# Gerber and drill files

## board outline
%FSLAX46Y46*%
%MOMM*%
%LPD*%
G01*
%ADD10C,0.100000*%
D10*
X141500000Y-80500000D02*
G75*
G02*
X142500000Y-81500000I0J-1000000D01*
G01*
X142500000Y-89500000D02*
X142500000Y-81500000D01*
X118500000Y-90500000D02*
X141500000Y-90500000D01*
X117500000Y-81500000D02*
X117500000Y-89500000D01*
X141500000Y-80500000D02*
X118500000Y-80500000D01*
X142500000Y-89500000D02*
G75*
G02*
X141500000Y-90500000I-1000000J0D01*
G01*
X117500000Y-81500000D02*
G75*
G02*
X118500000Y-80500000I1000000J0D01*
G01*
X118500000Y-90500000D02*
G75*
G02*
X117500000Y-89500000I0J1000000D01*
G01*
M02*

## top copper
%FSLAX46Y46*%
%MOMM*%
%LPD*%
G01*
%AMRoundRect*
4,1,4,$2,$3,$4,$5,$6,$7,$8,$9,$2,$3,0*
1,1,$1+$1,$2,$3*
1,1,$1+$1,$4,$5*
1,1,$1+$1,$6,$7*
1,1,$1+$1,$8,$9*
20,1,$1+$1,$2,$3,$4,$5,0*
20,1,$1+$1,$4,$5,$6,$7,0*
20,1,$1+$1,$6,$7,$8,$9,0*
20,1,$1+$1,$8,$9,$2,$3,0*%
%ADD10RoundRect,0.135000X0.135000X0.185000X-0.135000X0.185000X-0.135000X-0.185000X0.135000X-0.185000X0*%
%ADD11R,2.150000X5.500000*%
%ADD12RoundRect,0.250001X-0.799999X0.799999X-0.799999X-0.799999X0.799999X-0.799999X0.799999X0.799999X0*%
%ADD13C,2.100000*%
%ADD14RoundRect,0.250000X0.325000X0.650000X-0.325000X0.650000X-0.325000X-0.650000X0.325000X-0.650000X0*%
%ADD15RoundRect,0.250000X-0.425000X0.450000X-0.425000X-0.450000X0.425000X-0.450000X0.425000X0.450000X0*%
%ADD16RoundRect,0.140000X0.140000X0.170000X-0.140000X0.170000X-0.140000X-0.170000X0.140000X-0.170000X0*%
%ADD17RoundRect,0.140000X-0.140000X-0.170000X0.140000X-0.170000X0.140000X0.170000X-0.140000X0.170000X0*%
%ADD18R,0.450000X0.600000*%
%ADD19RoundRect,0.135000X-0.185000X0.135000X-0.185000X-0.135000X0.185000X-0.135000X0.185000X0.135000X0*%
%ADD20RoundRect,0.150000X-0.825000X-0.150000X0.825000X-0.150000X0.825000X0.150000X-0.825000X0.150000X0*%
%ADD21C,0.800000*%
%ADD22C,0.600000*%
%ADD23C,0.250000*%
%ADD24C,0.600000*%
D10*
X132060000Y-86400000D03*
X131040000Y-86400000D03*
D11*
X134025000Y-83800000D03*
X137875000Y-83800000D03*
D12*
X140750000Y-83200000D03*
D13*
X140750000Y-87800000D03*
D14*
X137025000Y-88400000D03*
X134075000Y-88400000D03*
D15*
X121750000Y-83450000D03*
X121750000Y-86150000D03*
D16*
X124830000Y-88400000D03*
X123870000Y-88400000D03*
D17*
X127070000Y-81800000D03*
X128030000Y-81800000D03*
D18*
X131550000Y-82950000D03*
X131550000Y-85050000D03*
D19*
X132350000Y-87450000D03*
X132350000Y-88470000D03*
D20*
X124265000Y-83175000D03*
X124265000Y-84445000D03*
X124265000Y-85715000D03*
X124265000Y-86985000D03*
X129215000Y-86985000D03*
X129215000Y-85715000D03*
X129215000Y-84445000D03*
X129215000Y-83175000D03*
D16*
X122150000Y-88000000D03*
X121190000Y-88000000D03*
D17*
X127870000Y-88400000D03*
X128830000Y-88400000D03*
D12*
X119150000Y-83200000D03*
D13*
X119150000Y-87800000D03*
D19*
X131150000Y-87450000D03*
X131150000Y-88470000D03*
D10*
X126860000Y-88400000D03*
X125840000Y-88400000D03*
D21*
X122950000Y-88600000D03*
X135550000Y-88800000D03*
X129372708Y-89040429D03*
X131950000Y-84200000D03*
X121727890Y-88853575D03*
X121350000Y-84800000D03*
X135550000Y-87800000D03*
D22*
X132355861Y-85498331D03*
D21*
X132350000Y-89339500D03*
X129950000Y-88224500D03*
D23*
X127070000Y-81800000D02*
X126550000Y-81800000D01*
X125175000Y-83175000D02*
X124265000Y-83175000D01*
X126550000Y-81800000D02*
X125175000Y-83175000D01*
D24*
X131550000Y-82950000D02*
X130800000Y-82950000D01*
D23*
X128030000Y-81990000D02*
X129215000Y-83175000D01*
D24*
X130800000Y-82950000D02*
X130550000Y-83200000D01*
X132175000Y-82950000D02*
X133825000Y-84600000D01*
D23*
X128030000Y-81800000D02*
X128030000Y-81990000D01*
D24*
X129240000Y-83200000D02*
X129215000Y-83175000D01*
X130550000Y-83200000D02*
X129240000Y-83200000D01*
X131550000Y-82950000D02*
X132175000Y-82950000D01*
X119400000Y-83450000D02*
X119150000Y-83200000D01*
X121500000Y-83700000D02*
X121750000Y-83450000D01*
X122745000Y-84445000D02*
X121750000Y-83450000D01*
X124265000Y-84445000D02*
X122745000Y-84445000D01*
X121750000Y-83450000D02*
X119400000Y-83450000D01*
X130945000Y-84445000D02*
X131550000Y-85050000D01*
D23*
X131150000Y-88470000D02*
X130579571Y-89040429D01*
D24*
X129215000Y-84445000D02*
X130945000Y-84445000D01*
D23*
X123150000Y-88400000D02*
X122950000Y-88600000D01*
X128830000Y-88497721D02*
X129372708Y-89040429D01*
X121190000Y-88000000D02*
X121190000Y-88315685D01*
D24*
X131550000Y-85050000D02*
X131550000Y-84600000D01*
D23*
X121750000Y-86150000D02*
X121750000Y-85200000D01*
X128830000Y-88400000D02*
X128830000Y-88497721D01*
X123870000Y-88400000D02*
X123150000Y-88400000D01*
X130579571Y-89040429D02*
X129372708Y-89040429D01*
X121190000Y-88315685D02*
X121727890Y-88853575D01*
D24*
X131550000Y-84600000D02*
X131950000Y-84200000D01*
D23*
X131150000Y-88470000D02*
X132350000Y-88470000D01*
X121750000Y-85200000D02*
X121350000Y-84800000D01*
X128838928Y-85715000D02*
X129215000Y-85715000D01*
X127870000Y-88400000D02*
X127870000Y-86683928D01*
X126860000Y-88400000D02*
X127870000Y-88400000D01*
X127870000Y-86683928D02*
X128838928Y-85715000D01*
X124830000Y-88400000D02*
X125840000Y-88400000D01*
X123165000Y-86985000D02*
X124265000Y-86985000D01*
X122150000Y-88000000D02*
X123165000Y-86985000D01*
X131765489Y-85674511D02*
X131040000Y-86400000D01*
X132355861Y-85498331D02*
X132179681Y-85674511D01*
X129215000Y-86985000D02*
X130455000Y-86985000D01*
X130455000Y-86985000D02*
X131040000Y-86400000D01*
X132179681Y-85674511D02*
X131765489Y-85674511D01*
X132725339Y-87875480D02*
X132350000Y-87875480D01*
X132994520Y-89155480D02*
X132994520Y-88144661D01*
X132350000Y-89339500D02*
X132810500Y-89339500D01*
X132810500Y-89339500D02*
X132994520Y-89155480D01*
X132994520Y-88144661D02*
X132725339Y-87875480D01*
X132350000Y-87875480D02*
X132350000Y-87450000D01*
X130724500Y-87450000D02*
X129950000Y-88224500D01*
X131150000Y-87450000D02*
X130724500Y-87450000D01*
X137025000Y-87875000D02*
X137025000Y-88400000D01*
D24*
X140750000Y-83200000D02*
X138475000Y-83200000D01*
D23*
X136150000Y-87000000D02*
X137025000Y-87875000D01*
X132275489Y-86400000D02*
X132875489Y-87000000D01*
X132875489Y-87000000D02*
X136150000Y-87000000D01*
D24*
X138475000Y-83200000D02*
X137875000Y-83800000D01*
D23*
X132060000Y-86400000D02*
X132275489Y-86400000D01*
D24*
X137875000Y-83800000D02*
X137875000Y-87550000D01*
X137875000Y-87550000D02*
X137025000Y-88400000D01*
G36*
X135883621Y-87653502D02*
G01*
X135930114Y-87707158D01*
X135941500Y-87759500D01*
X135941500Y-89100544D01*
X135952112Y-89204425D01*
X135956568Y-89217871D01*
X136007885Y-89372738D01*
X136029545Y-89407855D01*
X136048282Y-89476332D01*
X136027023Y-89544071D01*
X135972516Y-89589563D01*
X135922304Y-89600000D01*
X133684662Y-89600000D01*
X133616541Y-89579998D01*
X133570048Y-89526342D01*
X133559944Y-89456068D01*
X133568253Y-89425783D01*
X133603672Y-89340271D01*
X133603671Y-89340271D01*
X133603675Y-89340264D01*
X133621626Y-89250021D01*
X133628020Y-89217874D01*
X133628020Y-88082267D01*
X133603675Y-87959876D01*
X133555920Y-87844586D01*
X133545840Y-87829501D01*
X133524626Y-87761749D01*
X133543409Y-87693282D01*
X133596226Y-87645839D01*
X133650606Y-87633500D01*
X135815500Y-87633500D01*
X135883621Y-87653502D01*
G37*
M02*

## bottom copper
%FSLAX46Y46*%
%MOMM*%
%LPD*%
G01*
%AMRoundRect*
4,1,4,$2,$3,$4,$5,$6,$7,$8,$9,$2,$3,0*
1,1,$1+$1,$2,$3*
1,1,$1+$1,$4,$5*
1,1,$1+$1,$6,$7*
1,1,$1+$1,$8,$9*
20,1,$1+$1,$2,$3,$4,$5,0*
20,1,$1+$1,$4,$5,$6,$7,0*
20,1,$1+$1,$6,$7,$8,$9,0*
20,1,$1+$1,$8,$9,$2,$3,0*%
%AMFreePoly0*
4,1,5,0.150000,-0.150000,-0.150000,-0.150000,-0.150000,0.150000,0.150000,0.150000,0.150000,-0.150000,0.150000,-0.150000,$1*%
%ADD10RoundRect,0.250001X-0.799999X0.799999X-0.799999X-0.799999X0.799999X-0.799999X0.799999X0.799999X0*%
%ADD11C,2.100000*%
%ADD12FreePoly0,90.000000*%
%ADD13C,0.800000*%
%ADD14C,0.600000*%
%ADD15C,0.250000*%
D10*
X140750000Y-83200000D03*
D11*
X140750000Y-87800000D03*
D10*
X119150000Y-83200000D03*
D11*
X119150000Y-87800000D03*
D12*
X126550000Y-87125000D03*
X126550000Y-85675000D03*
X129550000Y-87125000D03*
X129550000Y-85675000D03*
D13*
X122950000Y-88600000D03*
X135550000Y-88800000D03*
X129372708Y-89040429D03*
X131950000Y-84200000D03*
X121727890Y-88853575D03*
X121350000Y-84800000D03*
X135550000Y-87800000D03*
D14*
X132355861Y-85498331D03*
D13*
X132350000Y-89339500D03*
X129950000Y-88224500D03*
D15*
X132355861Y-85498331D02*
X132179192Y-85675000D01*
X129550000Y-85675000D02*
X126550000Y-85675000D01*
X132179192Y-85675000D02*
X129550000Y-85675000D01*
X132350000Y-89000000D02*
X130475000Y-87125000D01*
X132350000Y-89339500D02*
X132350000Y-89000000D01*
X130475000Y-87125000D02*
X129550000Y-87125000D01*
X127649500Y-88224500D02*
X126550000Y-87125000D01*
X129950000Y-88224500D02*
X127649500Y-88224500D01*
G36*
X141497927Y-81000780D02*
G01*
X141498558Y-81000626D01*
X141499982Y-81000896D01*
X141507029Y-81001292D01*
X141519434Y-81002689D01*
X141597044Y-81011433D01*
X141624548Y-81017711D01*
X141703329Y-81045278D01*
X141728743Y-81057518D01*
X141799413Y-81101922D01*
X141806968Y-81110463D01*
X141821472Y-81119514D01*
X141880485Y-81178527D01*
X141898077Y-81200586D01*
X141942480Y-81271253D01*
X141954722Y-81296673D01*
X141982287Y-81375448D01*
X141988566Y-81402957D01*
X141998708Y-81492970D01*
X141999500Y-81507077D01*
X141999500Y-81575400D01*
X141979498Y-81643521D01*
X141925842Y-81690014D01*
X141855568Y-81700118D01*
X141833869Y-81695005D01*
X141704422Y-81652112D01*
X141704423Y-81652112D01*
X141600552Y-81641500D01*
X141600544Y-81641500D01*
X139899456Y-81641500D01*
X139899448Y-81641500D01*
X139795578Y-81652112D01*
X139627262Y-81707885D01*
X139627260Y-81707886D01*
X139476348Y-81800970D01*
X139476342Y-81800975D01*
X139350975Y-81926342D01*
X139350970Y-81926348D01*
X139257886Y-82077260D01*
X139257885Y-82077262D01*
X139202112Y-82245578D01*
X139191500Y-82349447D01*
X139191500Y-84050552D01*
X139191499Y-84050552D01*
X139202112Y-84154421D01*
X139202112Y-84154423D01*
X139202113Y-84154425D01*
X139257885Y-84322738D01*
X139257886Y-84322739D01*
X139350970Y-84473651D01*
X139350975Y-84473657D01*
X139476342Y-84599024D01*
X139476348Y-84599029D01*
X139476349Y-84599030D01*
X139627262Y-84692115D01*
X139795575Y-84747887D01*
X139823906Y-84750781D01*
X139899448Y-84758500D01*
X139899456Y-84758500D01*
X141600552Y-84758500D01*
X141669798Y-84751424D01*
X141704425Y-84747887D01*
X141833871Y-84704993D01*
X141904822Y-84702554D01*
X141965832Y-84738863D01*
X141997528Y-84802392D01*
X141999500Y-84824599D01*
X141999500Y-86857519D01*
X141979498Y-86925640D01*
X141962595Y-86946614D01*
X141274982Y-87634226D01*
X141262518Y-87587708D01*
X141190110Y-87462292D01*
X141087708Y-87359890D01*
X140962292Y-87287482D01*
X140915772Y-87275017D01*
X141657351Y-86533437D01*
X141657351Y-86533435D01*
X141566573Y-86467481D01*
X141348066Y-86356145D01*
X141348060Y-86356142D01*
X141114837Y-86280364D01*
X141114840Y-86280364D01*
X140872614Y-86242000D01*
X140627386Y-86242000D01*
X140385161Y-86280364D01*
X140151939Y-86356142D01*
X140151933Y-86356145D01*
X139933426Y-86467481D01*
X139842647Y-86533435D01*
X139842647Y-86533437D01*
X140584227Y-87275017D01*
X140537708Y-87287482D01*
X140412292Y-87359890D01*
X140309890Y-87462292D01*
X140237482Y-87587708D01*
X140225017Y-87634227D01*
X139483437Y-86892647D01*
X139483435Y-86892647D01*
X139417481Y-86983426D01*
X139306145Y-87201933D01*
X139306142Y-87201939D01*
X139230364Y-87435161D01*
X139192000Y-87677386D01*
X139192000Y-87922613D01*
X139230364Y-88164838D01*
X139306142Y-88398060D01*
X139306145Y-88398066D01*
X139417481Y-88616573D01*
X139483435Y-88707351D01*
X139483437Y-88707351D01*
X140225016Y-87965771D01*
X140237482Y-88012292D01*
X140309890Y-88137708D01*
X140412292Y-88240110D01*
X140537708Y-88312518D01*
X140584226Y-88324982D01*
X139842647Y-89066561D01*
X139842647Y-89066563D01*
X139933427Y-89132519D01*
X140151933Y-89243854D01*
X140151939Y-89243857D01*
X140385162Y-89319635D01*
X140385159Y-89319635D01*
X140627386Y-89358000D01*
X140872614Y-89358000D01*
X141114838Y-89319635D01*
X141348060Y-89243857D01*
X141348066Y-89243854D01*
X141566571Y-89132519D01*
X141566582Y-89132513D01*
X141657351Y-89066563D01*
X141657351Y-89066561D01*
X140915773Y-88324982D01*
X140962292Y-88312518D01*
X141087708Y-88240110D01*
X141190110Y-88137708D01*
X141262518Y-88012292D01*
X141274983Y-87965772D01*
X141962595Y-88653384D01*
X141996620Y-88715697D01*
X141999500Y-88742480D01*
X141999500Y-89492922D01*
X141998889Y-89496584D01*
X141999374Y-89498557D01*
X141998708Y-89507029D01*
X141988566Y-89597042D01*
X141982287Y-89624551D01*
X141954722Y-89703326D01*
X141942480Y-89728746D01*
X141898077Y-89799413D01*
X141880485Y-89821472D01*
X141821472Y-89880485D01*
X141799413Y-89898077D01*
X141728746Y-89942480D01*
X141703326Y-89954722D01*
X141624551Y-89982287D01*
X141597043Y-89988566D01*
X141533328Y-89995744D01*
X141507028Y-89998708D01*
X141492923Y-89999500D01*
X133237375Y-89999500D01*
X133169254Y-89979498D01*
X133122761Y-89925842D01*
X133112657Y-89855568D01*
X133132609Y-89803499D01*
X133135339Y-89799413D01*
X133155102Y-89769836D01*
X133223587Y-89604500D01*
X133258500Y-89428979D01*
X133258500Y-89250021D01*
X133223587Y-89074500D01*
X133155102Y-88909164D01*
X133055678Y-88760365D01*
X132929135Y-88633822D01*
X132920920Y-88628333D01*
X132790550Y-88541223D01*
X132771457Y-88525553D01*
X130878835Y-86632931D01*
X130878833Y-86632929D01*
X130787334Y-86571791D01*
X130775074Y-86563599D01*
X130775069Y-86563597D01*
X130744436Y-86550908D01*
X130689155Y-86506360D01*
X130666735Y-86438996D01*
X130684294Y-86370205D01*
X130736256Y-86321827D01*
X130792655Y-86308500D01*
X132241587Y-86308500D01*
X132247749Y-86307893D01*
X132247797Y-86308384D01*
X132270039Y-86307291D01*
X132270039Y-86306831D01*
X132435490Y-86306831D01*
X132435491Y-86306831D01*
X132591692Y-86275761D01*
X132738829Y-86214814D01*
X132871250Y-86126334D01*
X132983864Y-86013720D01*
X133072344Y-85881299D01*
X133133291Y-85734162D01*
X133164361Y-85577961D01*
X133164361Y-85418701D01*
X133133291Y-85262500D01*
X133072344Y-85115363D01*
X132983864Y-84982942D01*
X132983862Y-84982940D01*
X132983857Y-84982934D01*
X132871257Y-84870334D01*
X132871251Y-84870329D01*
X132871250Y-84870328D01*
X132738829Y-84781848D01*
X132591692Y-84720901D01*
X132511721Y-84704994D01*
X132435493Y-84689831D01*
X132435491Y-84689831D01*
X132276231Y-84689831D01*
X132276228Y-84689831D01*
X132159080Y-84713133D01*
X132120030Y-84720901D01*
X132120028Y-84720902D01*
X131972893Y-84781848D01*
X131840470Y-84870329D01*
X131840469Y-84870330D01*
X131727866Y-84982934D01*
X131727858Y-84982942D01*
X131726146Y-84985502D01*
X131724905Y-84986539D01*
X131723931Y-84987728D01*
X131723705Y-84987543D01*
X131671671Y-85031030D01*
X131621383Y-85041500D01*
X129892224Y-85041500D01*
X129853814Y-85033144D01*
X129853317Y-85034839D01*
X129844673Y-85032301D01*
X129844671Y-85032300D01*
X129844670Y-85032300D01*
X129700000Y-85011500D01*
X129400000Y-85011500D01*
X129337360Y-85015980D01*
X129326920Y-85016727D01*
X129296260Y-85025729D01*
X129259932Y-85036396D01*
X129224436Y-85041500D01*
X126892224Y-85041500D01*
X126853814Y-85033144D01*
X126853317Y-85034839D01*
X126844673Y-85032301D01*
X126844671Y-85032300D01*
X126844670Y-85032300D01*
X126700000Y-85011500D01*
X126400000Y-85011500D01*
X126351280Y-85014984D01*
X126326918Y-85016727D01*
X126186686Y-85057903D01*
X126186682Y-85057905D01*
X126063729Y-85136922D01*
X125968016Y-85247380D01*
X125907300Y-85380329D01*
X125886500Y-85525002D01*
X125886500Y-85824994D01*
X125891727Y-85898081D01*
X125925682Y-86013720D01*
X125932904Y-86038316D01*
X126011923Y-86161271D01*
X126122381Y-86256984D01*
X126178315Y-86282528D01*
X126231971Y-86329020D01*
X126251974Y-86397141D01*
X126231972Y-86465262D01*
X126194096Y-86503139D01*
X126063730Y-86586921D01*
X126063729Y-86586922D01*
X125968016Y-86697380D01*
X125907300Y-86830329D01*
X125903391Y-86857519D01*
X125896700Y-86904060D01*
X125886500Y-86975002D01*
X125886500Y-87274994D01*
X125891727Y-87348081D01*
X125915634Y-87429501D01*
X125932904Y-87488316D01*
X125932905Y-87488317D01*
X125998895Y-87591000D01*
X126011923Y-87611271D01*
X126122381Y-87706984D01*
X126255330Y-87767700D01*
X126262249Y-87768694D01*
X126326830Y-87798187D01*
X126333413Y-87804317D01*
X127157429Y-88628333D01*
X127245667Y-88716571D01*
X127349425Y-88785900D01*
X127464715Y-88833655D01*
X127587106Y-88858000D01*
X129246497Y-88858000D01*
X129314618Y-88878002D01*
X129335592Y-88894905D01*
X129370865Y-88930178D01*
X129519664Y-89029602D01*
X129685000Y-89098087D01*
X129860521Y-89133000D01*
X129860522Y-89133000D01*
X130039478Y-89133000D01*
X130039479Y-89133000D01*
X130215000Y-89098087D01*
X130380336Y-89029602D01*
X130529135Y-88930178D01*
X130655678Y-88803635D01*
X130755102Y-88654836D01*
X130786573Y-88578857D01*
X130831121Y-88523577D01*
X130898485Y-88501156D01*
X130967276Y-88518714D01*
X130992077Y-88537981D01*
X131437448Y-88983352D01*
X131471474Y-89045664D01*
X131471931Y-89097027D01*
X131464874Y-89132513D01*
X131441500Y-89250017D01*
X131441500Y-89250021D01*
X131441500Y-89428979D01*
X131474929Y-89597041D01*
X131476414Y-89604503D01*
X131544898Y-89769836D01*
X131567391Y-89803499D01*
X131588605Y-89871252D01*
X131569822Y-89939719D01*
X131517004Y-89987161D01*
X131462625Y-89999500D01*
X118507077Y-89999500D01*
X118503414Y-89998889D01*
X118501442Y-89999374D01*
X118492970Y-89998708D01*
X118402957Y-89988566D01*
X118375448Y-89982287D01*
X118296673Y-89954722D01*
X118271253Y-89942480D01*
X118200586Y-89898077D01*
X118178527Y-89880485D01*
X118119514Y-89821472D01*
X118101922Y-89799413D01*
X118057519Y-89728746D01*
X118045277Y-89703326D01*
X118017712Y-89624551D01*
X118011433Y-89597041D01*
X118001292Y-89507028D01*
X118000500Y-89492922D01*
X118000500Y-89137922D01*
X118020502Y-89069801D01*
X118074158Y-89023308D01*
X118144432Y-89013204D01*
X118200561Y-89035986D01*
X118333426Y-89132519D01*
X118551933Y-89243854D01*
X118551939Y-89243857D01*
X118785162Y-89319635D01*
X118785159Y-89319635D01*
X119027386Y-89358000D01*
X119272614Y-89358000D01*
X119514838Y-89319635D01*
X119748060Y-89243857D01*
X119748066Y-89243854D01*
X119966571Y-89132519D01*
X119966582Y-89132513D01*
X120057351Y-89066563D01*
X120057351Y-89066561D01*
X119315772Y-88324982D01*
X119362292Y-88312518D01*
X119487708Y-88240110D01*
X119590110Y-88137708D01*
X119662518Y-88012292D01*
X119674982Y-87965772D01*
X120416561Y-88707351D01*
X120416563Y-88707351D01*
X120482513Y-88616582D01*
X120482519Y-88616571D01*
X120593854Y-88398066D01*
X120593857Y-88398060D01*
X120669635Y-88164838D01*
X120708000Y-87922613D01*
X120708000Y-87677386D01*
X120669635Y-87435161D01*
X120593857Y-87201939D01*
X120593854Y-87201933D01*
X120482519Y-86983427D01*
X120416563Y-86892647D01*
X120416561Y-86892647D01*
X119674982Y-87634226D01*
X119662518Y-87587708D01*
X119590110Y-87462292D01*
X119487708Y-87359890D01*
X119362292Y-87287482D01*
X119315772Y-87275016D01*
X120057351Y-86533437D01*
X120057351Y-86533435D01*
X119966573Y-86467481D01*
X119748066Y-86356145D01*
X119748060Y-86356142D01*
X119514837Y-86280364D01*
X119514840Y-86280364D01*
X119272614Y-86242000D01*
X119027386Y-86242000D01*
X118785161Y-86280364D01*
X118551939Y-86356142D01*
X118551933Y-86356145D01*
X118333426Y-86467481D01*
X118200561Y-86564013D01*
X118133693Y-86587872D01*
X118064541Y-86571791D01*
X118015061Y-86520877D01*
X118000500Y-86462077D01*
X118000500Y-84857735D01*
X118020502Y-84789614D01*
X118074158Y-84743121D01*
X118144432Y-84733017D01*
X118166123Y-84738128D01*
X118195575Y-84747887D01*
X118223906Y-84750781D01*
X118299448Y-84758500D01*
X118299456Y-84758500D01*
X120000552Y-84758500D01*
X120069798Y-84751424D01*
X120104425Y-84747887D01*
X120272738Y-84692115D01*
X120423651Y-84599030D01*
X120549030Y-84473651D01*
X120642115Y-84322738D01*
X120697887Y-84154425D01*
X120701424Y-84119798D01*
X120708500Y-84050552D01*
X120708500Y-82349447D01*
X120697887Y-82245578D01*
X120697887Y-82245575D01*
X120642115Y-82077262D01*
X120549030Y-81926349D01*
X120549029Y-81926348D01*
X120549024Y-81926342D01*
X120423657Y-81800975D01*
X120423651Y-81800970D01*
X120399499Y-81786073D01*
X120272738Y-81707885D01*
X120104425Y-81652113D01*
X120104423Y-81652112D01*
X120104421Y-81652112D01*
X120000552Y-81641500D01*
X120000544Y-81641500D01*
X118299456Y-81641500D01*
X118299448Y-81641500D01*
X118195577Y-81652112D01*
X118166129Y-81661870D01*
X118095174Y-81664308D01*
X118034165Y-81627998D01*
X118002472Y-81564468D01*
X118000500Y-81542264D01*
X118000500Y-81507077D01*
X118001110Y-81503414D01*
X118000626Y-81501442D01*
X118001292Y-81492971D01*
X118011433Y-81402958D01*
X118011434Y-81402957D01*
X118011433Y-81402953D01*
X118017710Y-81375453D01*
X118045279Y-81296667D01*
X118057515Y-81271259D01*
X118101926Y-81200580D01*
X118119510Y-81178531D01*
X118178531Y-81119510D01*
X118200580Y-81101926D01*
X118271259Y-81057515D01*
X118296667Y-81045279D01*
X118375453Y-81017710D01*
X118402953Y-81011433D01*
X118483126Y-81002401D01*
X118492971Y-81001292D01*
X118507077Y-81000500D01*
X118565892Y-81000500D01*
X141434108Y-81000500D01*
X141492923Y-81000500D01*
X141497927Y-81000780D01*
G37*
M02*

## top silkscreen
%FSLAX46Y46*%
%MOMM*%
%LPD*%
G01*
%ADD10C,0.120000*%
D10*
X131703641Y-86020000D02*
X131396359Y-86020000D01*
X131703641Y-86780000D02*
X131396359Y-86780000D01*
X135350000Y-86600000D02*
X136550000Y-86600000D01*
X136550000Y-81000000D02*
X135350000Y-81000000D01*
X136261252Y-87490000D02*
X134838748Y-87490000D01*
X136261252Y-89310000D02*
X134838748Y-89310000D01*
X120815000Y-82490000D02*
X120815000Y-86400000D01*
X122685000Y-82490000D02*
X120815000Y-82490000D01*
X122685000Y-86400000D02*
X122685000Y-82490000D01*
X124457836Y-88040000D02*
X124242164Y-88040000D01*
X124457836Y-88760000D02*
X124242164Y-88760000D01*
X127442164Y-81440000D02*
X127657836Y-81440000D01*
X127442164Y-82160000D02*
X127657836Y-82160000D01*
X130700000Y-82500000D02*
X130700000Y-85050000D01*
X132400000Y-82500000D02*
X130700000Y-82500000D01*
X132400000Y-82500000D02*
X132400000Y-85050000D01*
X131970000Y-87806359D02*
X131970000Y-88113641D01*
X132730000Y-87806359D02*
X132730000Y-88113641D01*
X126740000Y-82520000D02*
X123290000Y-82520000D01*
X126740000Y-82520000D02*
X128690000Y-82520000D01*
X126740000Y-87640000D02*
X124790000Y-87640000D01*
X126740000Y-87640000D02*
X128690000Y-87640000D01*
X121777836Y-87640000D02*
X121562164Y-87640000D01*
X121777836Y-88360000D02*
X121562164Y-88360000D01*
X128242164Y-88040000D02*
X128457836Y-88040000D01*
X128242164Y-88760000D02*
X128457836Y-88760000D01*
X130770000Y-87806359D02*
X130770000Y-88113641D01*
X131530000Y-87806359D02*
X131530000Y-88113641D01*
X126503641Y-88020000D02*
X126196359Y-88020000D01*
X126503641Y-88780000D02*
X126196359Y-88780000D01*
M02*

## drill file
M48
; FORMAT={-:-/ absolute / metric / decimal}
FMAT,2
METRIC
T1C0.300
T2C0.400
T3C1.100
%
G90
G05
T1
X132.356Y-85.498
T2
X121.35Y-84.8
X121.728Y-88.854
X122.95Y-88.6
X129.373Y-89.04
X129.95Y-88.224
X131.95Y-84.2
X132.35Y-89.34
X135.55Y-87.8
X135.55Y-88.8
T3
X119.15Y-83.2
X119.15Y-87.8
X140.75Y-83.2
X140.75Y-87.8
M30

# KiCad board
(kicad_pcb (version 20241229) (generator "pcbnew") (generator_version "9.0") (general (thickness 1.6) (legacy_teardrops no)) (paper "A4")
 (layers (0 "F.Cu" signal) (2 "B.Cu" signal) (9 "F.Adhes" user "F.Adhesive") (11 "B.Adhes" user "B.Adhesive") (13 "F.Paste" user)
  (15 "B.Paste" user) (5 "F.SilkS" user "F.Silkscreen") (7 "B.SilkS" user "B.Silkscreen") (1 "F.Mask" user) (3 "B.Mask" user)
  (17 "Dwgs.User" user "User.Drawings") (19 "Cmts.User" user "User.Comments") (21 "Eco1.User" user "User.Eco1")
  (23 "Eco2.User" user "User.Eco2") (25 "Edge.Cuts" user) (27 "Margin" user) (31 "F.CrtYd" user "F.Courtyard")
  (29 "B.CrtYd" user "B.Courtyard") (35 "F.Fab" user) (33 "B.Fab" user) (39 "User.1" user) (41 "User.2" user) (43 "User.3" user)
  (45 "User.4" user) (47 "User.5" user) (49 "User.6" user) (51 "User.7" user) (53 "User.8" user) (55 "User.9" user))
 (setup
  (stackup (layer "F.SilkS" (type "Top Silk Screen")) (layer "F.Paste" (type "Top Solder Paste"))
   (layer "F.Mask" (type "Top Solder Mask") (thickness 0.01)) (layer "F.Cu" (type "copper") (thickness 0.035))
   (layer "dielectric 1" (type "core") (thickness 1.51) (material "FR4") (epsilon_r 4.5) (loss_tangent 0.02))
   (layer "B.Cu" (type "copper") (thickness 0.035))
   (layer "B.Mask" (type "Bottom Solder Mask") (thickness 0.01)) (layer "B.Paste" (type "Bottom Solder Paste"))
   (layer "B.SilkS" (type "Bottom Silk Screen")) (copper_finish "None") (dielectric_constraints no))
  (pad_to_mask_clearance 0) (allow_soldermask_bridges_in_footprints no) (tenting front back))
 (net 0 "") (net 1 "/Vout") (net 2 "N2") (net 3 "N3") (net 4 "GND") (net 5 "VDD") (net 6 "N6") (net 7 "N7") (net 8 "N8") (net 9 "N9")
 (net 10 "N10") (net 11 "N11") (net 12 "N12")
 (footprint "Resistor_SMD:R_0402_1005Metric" (layer "F.Cu") (at 131.55 86.4 180)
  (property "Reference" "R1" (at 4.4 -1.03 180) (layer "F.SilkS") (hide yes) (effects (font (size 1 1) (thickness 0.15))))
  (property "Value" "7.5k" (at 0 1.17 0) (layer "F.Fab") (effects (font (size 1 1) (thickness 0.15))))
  (fp_line (start -0.153641 0.38) (end 0.153641 0.38) (stroke (width 0.12) (type solid)) (layer "F.SilkS"))
  (fp_line (start -0.153641 -0.38) (end 0.153641 -0.38) (stroke (width 0.12) (type solid)) (layer "F.SilkS"))
  (pad "1" smd roundrect (at -0.51 0 180) (size 0.54 0.64) (layers "F.Cu" "F.Mask" "F.Paste") (roundrect_rratio 0.25) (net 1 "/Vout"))
  (pad "2" smd roundrect (at 0.51 0 180) (size 0.54 0.64) (layers "F.Cu" "F.Mask" "F.Paste") (roundrect_rratio 0.25) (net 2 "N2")))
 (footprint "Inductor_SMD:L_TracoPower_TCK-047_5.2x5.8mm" (layer "F.Cu") (at 135.95 83.8)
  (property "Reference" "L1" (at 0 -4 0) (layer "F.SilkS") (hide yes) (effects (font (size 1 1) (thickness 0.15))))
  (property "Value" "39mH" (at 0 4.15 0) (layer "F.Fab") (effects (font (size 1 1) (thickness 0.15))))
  (fp_line (start -0.6 2.8) (end 0.6 2.8) (stroke (width 0.12) (type solid)) (layer "F.SilkS"))
  (fp_line (start 0.6 -2.8) (end -0.6 -2.8) (stroke (width 0.12) (type solid)) (layer "F.SilkS"))
  (pad "1" smd rect (at -1.925 0 90) (size 5.5 2.15) (layers "F.Cu" "F.Mask" "F.Paste") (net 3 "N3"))
  (pad "2" smd rect (at 1.925 0 90) (size 5.5 2.15) (layers "F.Cu" "F.Mask" "F.Paste") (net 1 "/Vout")))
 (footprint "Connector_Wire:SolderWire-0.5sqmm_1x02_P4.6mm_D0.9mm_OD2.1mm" (layer "F.Cu") (at 140.75 83.2 -90)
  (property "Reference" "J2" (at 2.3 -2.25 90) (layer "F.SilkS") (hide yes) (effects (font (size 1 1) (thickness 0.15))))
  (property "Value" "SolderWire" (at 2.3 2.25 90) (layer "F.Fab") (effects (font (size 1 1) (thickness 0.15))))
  (pad "1" thru_hole roundrect (at 0 0 270) (size 2.1 2.1) (drill 1.1) (layers "*.Cu" "*.Mask") (remove_unused_layers no)
   (roundrect_rratio 0.1190480952) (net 1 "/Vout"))
  (pad "2" thru_hole circle (at 4.6 0 270) (size 2.1 2.1) (drill 1.1) (layers "*.Cu" "*.Mask") (remove_unused_layers no) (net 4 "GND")))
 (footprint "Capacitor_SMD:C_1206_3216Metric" (layer "F.Cu") (at 135.55 88.4 180)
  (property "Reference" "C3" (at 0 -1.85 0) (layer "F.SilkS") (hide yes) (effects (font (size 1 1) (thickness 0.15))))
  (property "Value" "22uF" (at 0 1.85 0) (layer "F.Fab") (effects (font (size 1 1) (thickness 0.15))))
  (fp_line (start -0.711252 0.91) (end 0.711252 0.91) (stroke (width 0.12) (type solid)) (layer "F.SilkS"))
  (fp_line (start -0.711252 -0.91) (end 0.711252 -0.91) (stroke (width 0.12) (type solid)) (layer "F.SilkS"))
  (pad "1" smd roundrect (at -1.475 0 180) (size 1.15 1.8) (layers "F.Cu" "F.Mask" "F.Paste") (roundrect_rratio 0.2173913043)
   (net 1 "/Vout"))
  (pad "2" smd roundrect (at 1.475 0 180) (size 1.15 1.8) (layers "F.Cu" "F.Mask" "F.Paste") (roundrect_rratio 0.2173913043) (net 4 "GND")))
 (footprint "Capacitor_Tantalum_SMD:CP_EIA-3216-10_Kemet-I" (layer "F.Cu") (at 121.75 84.8 -90)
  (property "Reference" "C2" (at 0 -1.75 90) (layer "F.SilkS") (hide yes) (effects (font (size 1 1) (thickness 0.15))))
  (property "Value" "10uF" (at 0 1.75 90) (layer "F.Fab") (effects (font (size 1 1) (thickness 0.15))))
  (fp_line (start -2.31 0.935) (end 1.6 0.935) (stroke (width 0.12) (type solid)) (layer "F.SilkS"))
  (fp_line (start -2.31 -0.935) (end -2.31 0.935) (stroke (width 0.12) (type solid)) (layer "F.SilkS"))
  (fp_line (start 1.6 -0.935) (end -2.31 -0.935) (stroke (width 0.12) (type solid)) (layer "F.SilkS"))
  (pad "1" smd roundrect (at -1.35 0 270) (size 1.4 1.35) (layers "F.Cu" "F.Mask" "F.Paste") (roundrect_rratio 0.1851851852) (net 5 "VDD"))
  (pad "2" smd roundrect (at 1.35 0 270) (size 1.4 1.35) (layers "F.Cu" "F.Mask" "F.Paste") (roundrect_rratio 0.1851851852) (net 4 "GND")))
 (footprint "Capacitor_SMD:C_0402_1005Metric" (layer "F.Cu") (at 124.35 88.4 180)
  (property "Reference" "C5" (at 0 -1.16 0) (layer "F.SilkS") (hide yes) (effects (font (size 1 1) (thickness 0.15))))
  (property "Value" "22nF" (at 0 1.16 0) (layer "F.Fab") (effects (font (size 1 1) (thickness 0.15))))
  (fp_line (start -0.107836 0.36) (end 0.107836 0.36) (stroke (width 0.12) (type solid)) (layer "F.SilkS"))
  (fp_line (start -0.107836 -0.36) (end 0.107836 -0.36) (stroke (width 0.12) (type solid)) (layer "F.SilkS"))
  (pad "1" smd roundrect (at -0.48 0 180) (size 0.56 0.62) (layers "F.Cu" "F.Mask" "F.Paste") (roundrect_rratio 0.25) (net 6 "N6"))
  (pad "2" smd roundrect (at 0.48 0 180) (size 0.56 0.62) (layers "F.Cu" "F.Mask" "F.Paste") (roundrect_rratio 0.25) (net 4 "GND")))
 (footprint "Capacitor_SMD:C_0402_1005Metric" (layer "F.Cu") (at 127.55 81.8)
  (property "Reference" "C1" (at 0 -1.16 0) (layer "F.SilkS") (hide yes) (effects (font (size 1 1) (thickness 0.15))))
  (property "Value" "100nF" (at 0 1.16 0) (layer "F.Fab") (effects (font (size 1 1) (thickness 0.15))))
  (fp_line (start -0.107836 -0.36) (end 0.107836 -0.36) (stroke (width 0.12) (type solid)) (layer "F.SilkS"))
  (fp_line (start -0.107836 0.36) (end 0.107836 0.36) (stroke (width 0.12) (type solid)) (layer "F.SilkS"))
  (pad "1" smd roundrect (at -0.48 0) (size 0.56 0.62) (layers "F.Cu" "F.Mask" "F.Paste") (roundrect_rratio 0.25) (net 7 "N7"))
  (pad "2" smd roundrect (at 0.48 0) (size 0.56 0.62) (layers "F.Cu" "F.Mask" "F.Paste") (roundrect_rratio 0.25) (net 3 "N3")))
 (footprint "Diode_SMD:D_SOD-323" (layer "F.Cu") (at 131.55 84 -90)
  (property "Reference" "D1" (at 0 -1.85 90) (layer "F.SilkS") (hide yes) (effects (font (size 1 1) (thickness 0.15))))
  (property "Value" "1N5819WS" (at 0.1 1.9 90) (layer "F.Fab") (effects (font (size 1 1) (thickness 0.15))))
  (fp_line (start -1.5 0.85) (end 1.05 0.85) (stroke (width 0.12) (type solid)) (layer "F.SilkS"))
  (fp_line (start -1.5 -0.85) (end -1.5 0.85) (stroke (width 0.12) (type solid)) (layer "F.SilkS"))
  (fp_line (start -1.5 -0.85) (end 1.05 -0.85) (stroke (width 0.12) (type solid)) (layer "F.SilkS"))
  (pad "1" smd rect (at -1.05 0 270) (size 0.6 0.45) (layers "F.Cu" "F.Mask" "F.Paste") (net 3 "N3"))
  (pad "2" smd rect (at 1.05 0 270) (size 0.6 0.45) (layers "F.Cu" "F.Mask" "F.Paste") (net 4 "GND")))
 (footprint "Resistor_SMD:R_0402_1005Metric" (layer "F.Cu") (at 132.35 87.96 -90)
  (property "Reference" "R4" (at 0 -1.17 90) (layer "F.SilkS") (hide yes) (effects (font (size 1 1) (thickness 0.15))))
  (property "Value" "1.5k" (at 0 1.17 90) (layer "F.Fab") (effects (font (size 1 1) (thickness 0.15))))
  (fp_line (start -0.153641 0.38) (end 0.153641 0.38) (stroke (width 0.12) (type solid)) (layer "F.SilkS"))
  (fp_line (start -0.153641 -0.38) (end 0.153641 -0.38) (stroke (width 0.12) (type solid)) (layer "F.SilkS"))
  (pad "1" smd roundrect (at -0.51 0 270) (size 0.54 0.64) (layers "F.Cu" "F.Mask" "F.Paste") (roundrect_rratio 0.25) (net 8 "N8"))
  (pad "2" smd roundrect (at 0.51 0 270) (size 0.54 0.64) (layers "F.Cu" "F.Mask" "F.Paste") (roundrect_rratio 0.25) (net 4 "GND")))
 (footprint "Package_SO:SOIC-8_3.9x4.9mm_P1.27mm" (layer "F.Cu") (at 126.74 85.08 90)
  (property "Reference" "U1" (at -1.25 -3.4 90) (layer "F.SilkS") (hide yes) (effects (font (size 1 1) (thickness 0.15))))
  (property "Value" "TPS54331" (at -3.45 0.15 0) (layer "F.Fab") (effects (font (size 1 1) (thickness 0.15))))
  (fp_line (start 2.56 0) (end 2.56 -3.45) (stroke (width 0.12) (type solid)) (layer "F.SilkS"))
  (fp_line (start 2.56 0) (end 2.56 1.95) (stroke (width 0.12) (type solid)) (layer "F.SilkS"))
  (fp_line (start -2.56 0) (end -2.56 -1.95) (stroke (width 0.12) (type solid)) (layer "F.SilkS"))
  (fp_line (start -2.56 0) (end -2.56 1.95) (stroke (width 0.12) (type solid)) (layer "F.SilkS"))
  (pad "1" smd roundrect (at 1.905 -2.475) (size 1.95 0.6) (layers "F.Cu" "F.Mask" "F.Paste") (roundrect_rratio 0.25) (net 7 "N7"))
  (pad "2" smd roundrect (at 0.635 -2.475) (size 1.95 0.6) (layers "F.Cu" "F.Mask" "F.Paste") (roundrect_rratio 0.25) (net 5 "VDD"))
  (pad "3" smd roundrect (at -0.635 -2.475) (size 1.95 0.6) (layers "F.Cu" "F.Mask" "F.Paste") (roundrect_rratio 0.25) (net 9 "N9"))
  (pad "4" smd roundrect (at -1.905 -2.475) (size 1.95 0.6) (layers "F.Cu" "F.Mask" "F.Paste") (roundrect_rratio 0.25) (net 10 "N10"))
  (pad "5" smd roundrect (at -1.905 2.475) (size 1.95 0.6) (layers "F.Cu" "F.Mask" "F.Paste") (roundrect_rratio 0.25) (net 2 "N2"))
  (pad "6" smd roundrect (at -0.635 2.475) (size 1.95 0.6) (layers "F.Cu" "F.Mask" "F.Paste") (roundrect_rratio 0.25) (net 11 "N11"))
  (pad "7" smd roundrect (at 0.635 2.475) (size 1.95 0.6) (layers "F.Cu" "F.Mask" "F.Paste") (roundrect_rratio 0.25) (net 4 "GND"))
  (pad "8" smd roundrect (at 1.905 2.475) (size 1.95 0.6) (layers "F.Cu" "F.Mask" "F.Paste") (roundrect_rratio 0.25) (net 3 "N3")))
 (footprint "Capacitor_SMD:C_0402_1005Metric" (layer "F.Cu") (at 121.67 88 180)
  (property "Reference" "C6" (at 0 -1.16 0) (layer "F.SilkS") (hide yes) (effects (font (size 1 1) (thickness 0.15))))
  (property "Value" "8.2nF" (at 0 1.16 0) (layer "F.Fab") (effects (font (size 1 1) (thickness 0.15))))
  (fp_line (start -0.107836 0.36) (end 0.107836 0.36) (stroke (width 0.12) (type solid)) (layer "F.SilkS"))
  (fp_line (start -0.107836 -0.36) (end 0.107836 -0.36) (stroke (width 0.12) (type solid)) (layer "F.SilkS"))
  (pad "1" smd roundrect (at -0.48 0 180) (size 0.56 0.62) (layers "F.Cu" "F.Mask" "F.Paste") (roundrect_rratio 0.25) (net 10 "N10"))
  (pad "2" smd roundrect (at 0.48 0 180) (size 0.56 0.62) (layers "F.Cu" "F.Mask" "F.Paste") (roundrect_rratio 0.25) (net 4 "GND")))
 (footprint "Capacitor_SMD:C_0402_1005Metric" (layer "F.Cu") (at 128.35 88.4)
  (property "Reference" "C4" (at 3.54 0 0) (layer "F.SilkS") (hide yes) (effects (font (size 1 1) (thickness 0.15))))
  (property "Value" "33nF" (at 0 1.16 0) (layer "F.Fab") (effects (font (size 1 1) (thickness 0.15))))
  (fp_line (start -0.107836 -0.36) (end 0.107836 -0.36) (stroke (width 0.12) (type solid)) (layer "F.SilkS"))
  (fp_line (start -0.107836 0.36) (end 0.107836 0.36) (stroke (width 0.12) (type solid)) (layer "F.SilkS"))
  (pad "1" smd roundrect (at -0.48 0) (size 0.56 0.62) (layers "F.Cu" "F.Mask" "F.Paste") (roundrect_rratio 0.25) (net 11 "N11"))
  (pad "2" smd roundrect (at 0.48 0) (size 0.56 0.62) (layers "F.Cu" "F.Mask" "F.Paste") (roundrect_rratio 0.25) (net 4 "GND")))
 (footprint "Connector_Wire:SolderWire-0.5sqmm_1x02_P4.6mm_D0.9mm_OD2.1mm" (layer "F.Cu") (at 119.15 83.2 -90)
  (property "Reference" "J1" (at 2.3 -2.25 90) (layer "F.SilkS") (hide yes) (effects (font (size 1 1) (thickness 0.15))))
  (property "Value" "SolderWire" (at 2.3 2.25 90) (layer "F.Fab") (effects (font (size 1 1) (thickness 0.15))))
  (pad "1" thru_hole roundrect (at 0 0 270) (size 2.1 2.1) (drill 1.1) (layers "*.Cu" "*.Mask") (remove_unused_layers no)
   (roundrect_rratio 0.1190480952) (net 5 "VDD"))
  (pad "2" thru_hole circle (at 4.6 0 270) (size 2.1 2.1) (drill 1.1) (layers "*.Cu" "*.Mask") (remove_unused_layers no) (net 4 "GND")))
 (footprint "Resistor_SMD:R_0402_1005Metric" (layer "F.Cu") (at 131.15 87.96 -90)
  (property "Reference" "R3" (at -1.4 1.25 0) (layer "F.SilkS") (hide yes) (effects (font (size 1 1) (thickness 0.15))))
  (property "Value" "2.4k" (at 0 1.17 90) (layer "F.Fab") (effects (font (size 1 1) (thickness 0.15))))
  (fp_line (start -0.153641 0.38) (end 0.153641 0.38) (stroke (width 0.12) (type solid)) (layer "F.SilkS"))
  (fp_line (start -0.153641 -0.38) (end 0.153641 -0.38) (stroke (width 0.12) (type solid)) (layer "F.SilkS"))
  (pad "1" smd roundrect (at -0.51 0 270) (size 0.54 0.64) (layers "F.Cu" "F.Mask" "F.Paste") (roundrect_rratio 0.25) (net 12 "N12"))
  (pad "2" smd roundrect (at 0.51 0 270) (size 0.54 0.64) (layers "F.Cu" "F.Mask" "F.Paste") (roundrect_rratio 0.25) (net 4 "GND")))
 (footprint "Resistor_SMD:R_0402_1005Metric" (layer "F.Cu") (at 126.35 88.4 180)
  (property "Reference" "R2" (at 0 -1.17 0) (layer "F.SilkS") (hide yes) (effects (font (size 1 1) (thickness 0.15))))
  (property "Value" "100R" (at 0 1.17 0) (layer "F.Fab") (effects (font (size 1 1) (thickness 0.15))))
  (fp_line (start -0.153641 0.38) (end 0.153641 0.38) (stroke (width 0.12) (type solid)) (layer "F.SilkS"))
  (fp_line (start -0.153641 -0.38) (end 0.153641 -0.38) (stroke (width 0.12) (type solid)) (layer "F.SilkS"))
  (pad "1" smd roundrect (at -0.51 0 180) (size 0.54 0.64) (layers "F.Cu" "F.Mask" "F.Paste") (roundrect_rratio 0.25) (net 11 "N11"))
  (pad "2" smd roundrect (at 0.51 0 180) (size 0.54 0.64) (layers "F.Cu" "F.Mask" "F.Paste") (roundrect_rratio 0.25) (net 6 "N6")))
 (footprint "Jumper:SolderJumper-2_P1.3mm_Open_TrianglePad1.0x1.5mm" (layer "B.Cu") (at 126.55 86.4 90)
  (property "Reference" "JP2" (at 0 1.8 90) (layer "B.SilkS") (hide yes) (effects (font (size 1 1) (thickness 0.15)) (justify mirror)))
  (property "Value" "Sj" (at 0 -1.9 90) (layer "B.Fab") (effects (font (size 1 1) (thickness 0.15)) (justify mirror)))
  (pad "1" smd custom (at -0.725 0 90) (size 0.3 0.3) (layers "B.Cu" "B.Mask") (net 12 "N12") (zone_connect 2)
   (options (clearance outline) (anchor rect)) (primitives))
  (pad "2" smd custom (at 0.725 0 90) (size 0.3 0.3) (layers "B.Cu" "B.Mask") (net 2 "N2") (zone_connect 2)
   (options (clearance outline) (anchor rect)) (primitives)))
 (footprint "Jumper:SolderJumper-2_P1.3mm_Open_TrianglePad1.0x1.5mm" (layer "B.Cu") (at 129.55 86.4 90)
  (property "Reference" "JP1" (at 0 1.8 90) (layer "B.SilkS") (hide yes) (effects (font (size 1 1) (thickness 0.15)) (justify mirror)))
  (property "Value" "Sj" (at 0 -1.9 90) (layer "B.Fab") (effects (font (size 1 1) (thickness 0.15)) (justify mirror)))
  (pad "1" smd custom (at -0.725 0 90) (size 0.3 0.3) (layers "B.Cu" "B.Mask") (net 8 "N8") (zone_connect 2)
   (options (clearance outline) (anchor rect)) (primitives))
  (pad "2" smd custom (at 0.725 0 90) (size 0.3 0.3) (layers "B.Cu" "B.Mask") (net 2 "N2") (zone_connect 2)
   (options (clearance outline) (anchor rect)) (primitives)))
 (gr_arc (start 141.5 80.5) (mid 142.207107 80.792893) (end 142.5 81.5) (stroke (width 0.1) (type solid)) (layer "Edge.Cuts"))
 (gr_line (start 142.5 89.5) (end 142.5 81.5) (stroke (width 0.1) (type solid)) (layer "Edge.Cuts"))
 (gr_line (start 118.5 90.5) (end 141.5 90.5) (stroke (width 0.1) (type solid)) (layer "Edge.Cuts"))
 (gr_line (start 117.5 81.5) (end 117.5 89.5) (stroke (width 0.1) (type solid)) (layer "Edge.Cuts"))
 (gr_line (start 141.5 80.5) (end 118.5 80.5) (stroke (width 0.1) (type solid)) (layer "Edge.Cuts"))
 (gr_arc (start 142.5 89.5) (mid 142.207107 90.207107) (end 141.5 90.5) (stroke (width 0.1) (type solid)) (layer "Edge.Cuts"))
 (gr_arc (start 117.5 81.5) (mid 117.792893 80.792893) (end 118.5 80.5) (stroke (width 0.1) (type solid)) (layer "Edge.Cuts"))
 (gr_arc (start 118.5 90.5) (mid 117.792893 90.207107) (end 117.5 89.5) (stroke (width 0.1) (type solid)) (layer "Edge.Cuts"))
 (segment (start 127.07 81.8) (end 126.55 81.8) (width 0.25) (layer "F.Cu") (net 7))
 (segment (start 125.175 83.175) (end 124.265 83.175) (width 0.25) (layer "F.Cu") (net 7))
 (segment (start 126.55 81.8) (end 125.175 83.175) (width 0.25) (layer "F.Cu") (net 7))
 (segment (start 131.55 82.95) (end 130.8 82.95) (width 0.6) (layer "F.Cu") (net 3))
 (segment (start 128.03 81.99) (end 129.215 83.175) (width 0.25) (layer "F.Cu") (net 3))
 (segment (start 130.8 82.95) (end 130.55 83.2) (width 0.6) (layer "F.Cu") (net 3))
 (segment (start 132.175 82.95) (end 133.825 84.6) (width 0.6) (layer "F.Cu") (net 3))
 (segment (start 128.03 81.8) (end 128.03 81.99) (width 0.25) (layer "F.Cu") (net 3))
 (segment (start 129.24 83.2) (end 129.215 83.175) (width 0.6) (layer "F.Cu") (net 3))
 (segment (start 130.55 83.2) (end 129.24 83.2) (width 0.6) (layer "F.Cu") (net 3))
 (segment (start 131.55 82.95) (end 132.175 82.95) (width 0.6) (layer "F.Cu") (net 3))
 (segment (start 119.4 83.45) (end 119.15 83.2) (width 0.6) (layer "F.Cu") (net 5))
 (segment (start 121.5 83.7) (end 121.75 83.45) (width 0.6) (layer "F.Cu") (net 5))
 (segment (start 122.745 84.445) (end 121.75 83.45) (width 0.6) (layer "F.Cu") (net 5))
 (segment (start 124.265 84.445) (end 122.745 84.445) (width 0.6) (layer "F.Cu") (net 5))
 (segment (start 121.75 83.45) (end 119.4 83.45) (width 0.6) (layer "F.Cu") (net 5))
 (segment (start 130.945 84.445) (end 131.55 85.05) (width 0.6) (layer "F.Cu") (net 4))
 (segment (start 131.15 88.47) (end 130.579571 89.040429) (width 0.25) (layer "F.Cu") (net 4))
 (segment (start 129.215 84.445) (end 130.945 84.445) (width 0.6) (layer "F.Cu") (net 4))
 (segment (start 123.15 88.4) (end 122.95 88.6) (width 0.25) (layer "F.Cu") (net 4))
 (segment (start 128.83 88.497721) (end 129.372708 89.040429) (width 0.25) (layer "F.Cu") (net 4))
 (segment (start 121.19 88) (end 121.19 88.315685) (width 0.25) (layer "F.Cu") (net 4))
 (segment (start 131.55 85.05) (end 131.55 84.6) (width 0.6) (layer "F.Cu") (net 4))
 (segment (start 121.75 86.15) (end 121.75 85.2) (width 0.25) (layer "F.Cu") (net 4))
 (segment (start 128.83 88.4) (end 128.83 88.497721) (width 0.25) (layer "F.Cu") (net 4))
 (segment (start 123.87 88.4) (end 123.15 88.4) (width 0.25) (layer "F.Cu") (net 4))
 (segment (start 130.579571 89.040429) (end 129.372708 89.040429) (width 0.25) (layer "F.Cu") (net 4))
 (segment (start 121.19 88.315685) (end 121.72789 88.853575) (width 0.25) (layer "F.Cu") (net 4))
 (segment (start 131.55 84.6) (end 131.95 84.2) (width 0.6) (layer "F.Cu") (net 4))
 (segment (start 131.15 88.47) (end 132.35 88.47) (width 0.25) (layer "F.Cu") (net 4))
 (segment (start 121.75 85.2) (end 121.35 84.8) (width 0.25) (layer "F.Cu") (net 4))
 (via (at 122.95 88.6) (size 0.8) (drill 0.4) (layers "F.Cu" "B.Cu") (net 4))
 (via (at 135.55 88.8) (size 0.8) (drill 0.4) (layers "F.Cu" "B.Cu") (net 4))
 (via (at 129.372708 89.040429) (size 0.8) (drill 0.4) (layers "F.Cu" "B.Cu") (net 4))
 (via (at 131.95 84.2) (size 0.8) (drill 0.4) (layers "F.Cu" "B.Cu") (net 4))
 (via (at 121.72789 88.853575) (size 0.8) (drill 0.4) (layers "F.Cu" "B.Cu") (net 4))
 (via (at 121.35 84.8) (size 0.8) (drill 0.4) (layers "F.Cu" "B.Cu") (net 4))
 (via (at 135.55 87.8) (size 0.8) (drill 0.4) (layers "F.Cu" "B.Cu") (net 4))
 (segment (start 128.838928 85.715) (end 129.215 85.715) (width 0.25) (layer "F.Cu") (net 11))
 (segment (start 127.87 88.4) (end 127.87 86.683928) (width 0.25) (layer "F.Cu") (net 11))
 (segment (start 126.86 88.4) (end 127.87 88.4) (width 0.25) (layer "F.Cu") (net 11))
 (segment (start 127.87 86.683928) (end 128.838928 85.715) (width 0.25) (layer "F.Cu") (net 11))
 (segment (start 124.83 88.4) (end 125.84 88.4) (width 0.25) (layer "F.Cu") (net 6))
 (segment (start 123.165 86.985) (end 124.265 86.985) (width 0.25) (layer "F.Cu") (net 10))
 (segment (start 122.15 88) (end 123.165 86.985) (width 0.25) (layer "F.Cu") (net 10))
 (segment (start 131.765489 85.674511) (end 131.04 86.4) (width 0.25) (layer "F.Cu") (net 2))
 (segment (start 132.355861 85.498331) (end 132.179681 85.674511) (width 0.25) (layer "F.Cu") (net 2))
 (segment (start 129.215 86.985) (end 130.455 86.985) (width 0.25) (layer "F.Cu") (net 2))
 (segment (start 130.455 86.985) (end 131.04 86.4) (width 0.25) (layer "F.Cu") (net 2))
 (segment (start 132.179681 85.674511) (end 131.765489 85.674511) (width 0.25) (layer "F.Cu") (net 2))
 (via (at 132.355861 85.498331) (size 0.6) (drill 0.3) (layers "F.Cu" "B.Cu") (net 2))
 (segment (start 132.355861 85.498331) (end 132.179192 85.675) (width 0.25) (layer "B.Cu") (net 2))
 (segment (start 129.55 85.675) (end 126.55 85.675) (width 0.25) (layer "B.Cu") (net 2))
 (segment (start 132.179192 85.675) (end 129.55 85.675) (width 0.25) (layer "B.Cu") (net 2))
 (segment (start 132.725339 87.87548) (end 132.35 87.87548) (width 0.25) (layer "F.Cu") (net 8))
 (segment (start 132.99452 89.15548) (end 132.99452 88.144661) (width 0.25) (layer "F.Cu") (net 8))
 (segment (start 132.35 89.3395) (end 132.8105 89.3395) (width 0.25) (layer "F.Cu") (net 8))
 (segment (start 132.8105 89.3395) (end 132.99452 89.15548) (width 0.25) (layer "F.Cu") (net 8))
 (segment (start 132.99452 88.144661) (end 132.725339 87.87548) (width 0.25) (layer "F.Cu") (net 8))
 (segment (start 132.35 87.87548) (end 132.35 87.45) (width 0.25) (layer "F.Cu") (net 8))
 (via (at 132.35 89.3395) (size 0.8) (drill 0.4) (layers "F.Cu" "B.Cu") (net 8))
 (segment (start 132.35 89) (end 130.475 87.125) (width 0.25) (layer "B.Cu") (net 8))
 (segment (start 132.35 89.3395) (end 132.35 89) (width 0.25) (layer "B.Cu") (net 8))
 (segment (start 130.475 87.125) (end 129.55 87.125) (width 0.25) (layer "B.Cu") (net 8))
 (segment (start 130.7245 87.45) (end 129.95 88.2245) (width 0.25) (layer "F.Cu") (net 12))
 (segment (start 131.15 87.45) (end 130.7245 87.45) (width 0.25) (layer "F.Cu") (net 12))
 (via (at 129.95 88.2245) (size 0.8) (drill 0.4) (layers "F.Cu" "B.Cu") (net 12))
 (segment (start 127.6495 88.2245) (end 126.55 87.125) (width 0.25) (layer "B.Cu") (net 12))
 (segment (start 129.95 88.2245) (end 127.6495 88.2245) (width 0.25) (layer "B.Cu") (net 12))
 (segment (start 137.025 87.875) (end 137.025 88.4) (width 0.25) (layer "F.Cu") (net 1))
 (segment (start 140.75 83.2) (end 138.475 83.2) (width 0.6) (layer "F.Cu") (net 1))
 (segment (start 136.15 87) (end 137.025 87.875) (width 0.25) (layer "F.Cu") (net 1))
 (segment (start 132.275489 86.4) (end 132.875489 87) (width 0.25) (layer "F.Cu") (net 1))
 (segment (start 132.875489 87) (end 136.15 87) (width 0.25) (layer "F.Cu") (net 1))
 (segment (start 138.475 83.2) (end 137.875 83.8) (width 0.6) (layer "F.Cu") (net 1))
 (segment (start 132.06 86.4) (end 132.275489 86.4) (width 0.25) (layer "F.Cu") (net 1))
 (segment (start 137.875 83.8) (end 137.875 87.55) (width 0.6) (layer "F.Cu") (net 1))
 (segment (start 137.875 87.55) (end 137.025 88.4) (width 0.6) (layer "F.Cu") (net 1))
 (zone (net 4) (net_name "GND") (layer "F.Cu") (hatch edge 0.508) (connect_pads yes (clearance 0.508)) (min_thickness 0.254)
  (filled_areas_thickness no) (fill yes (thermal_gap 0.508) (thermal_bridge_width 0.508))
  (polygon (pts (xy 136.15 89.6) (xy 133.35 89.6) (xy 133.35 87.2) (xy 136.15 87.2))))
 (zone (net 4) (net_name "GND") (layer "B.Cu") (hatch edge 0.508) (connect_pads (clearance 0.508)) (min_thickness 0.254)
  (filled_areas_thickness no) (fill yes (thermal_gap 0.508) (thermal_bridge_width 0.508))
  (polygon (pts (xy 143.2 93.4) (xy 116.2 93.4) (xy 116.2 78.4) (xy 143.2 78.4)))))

